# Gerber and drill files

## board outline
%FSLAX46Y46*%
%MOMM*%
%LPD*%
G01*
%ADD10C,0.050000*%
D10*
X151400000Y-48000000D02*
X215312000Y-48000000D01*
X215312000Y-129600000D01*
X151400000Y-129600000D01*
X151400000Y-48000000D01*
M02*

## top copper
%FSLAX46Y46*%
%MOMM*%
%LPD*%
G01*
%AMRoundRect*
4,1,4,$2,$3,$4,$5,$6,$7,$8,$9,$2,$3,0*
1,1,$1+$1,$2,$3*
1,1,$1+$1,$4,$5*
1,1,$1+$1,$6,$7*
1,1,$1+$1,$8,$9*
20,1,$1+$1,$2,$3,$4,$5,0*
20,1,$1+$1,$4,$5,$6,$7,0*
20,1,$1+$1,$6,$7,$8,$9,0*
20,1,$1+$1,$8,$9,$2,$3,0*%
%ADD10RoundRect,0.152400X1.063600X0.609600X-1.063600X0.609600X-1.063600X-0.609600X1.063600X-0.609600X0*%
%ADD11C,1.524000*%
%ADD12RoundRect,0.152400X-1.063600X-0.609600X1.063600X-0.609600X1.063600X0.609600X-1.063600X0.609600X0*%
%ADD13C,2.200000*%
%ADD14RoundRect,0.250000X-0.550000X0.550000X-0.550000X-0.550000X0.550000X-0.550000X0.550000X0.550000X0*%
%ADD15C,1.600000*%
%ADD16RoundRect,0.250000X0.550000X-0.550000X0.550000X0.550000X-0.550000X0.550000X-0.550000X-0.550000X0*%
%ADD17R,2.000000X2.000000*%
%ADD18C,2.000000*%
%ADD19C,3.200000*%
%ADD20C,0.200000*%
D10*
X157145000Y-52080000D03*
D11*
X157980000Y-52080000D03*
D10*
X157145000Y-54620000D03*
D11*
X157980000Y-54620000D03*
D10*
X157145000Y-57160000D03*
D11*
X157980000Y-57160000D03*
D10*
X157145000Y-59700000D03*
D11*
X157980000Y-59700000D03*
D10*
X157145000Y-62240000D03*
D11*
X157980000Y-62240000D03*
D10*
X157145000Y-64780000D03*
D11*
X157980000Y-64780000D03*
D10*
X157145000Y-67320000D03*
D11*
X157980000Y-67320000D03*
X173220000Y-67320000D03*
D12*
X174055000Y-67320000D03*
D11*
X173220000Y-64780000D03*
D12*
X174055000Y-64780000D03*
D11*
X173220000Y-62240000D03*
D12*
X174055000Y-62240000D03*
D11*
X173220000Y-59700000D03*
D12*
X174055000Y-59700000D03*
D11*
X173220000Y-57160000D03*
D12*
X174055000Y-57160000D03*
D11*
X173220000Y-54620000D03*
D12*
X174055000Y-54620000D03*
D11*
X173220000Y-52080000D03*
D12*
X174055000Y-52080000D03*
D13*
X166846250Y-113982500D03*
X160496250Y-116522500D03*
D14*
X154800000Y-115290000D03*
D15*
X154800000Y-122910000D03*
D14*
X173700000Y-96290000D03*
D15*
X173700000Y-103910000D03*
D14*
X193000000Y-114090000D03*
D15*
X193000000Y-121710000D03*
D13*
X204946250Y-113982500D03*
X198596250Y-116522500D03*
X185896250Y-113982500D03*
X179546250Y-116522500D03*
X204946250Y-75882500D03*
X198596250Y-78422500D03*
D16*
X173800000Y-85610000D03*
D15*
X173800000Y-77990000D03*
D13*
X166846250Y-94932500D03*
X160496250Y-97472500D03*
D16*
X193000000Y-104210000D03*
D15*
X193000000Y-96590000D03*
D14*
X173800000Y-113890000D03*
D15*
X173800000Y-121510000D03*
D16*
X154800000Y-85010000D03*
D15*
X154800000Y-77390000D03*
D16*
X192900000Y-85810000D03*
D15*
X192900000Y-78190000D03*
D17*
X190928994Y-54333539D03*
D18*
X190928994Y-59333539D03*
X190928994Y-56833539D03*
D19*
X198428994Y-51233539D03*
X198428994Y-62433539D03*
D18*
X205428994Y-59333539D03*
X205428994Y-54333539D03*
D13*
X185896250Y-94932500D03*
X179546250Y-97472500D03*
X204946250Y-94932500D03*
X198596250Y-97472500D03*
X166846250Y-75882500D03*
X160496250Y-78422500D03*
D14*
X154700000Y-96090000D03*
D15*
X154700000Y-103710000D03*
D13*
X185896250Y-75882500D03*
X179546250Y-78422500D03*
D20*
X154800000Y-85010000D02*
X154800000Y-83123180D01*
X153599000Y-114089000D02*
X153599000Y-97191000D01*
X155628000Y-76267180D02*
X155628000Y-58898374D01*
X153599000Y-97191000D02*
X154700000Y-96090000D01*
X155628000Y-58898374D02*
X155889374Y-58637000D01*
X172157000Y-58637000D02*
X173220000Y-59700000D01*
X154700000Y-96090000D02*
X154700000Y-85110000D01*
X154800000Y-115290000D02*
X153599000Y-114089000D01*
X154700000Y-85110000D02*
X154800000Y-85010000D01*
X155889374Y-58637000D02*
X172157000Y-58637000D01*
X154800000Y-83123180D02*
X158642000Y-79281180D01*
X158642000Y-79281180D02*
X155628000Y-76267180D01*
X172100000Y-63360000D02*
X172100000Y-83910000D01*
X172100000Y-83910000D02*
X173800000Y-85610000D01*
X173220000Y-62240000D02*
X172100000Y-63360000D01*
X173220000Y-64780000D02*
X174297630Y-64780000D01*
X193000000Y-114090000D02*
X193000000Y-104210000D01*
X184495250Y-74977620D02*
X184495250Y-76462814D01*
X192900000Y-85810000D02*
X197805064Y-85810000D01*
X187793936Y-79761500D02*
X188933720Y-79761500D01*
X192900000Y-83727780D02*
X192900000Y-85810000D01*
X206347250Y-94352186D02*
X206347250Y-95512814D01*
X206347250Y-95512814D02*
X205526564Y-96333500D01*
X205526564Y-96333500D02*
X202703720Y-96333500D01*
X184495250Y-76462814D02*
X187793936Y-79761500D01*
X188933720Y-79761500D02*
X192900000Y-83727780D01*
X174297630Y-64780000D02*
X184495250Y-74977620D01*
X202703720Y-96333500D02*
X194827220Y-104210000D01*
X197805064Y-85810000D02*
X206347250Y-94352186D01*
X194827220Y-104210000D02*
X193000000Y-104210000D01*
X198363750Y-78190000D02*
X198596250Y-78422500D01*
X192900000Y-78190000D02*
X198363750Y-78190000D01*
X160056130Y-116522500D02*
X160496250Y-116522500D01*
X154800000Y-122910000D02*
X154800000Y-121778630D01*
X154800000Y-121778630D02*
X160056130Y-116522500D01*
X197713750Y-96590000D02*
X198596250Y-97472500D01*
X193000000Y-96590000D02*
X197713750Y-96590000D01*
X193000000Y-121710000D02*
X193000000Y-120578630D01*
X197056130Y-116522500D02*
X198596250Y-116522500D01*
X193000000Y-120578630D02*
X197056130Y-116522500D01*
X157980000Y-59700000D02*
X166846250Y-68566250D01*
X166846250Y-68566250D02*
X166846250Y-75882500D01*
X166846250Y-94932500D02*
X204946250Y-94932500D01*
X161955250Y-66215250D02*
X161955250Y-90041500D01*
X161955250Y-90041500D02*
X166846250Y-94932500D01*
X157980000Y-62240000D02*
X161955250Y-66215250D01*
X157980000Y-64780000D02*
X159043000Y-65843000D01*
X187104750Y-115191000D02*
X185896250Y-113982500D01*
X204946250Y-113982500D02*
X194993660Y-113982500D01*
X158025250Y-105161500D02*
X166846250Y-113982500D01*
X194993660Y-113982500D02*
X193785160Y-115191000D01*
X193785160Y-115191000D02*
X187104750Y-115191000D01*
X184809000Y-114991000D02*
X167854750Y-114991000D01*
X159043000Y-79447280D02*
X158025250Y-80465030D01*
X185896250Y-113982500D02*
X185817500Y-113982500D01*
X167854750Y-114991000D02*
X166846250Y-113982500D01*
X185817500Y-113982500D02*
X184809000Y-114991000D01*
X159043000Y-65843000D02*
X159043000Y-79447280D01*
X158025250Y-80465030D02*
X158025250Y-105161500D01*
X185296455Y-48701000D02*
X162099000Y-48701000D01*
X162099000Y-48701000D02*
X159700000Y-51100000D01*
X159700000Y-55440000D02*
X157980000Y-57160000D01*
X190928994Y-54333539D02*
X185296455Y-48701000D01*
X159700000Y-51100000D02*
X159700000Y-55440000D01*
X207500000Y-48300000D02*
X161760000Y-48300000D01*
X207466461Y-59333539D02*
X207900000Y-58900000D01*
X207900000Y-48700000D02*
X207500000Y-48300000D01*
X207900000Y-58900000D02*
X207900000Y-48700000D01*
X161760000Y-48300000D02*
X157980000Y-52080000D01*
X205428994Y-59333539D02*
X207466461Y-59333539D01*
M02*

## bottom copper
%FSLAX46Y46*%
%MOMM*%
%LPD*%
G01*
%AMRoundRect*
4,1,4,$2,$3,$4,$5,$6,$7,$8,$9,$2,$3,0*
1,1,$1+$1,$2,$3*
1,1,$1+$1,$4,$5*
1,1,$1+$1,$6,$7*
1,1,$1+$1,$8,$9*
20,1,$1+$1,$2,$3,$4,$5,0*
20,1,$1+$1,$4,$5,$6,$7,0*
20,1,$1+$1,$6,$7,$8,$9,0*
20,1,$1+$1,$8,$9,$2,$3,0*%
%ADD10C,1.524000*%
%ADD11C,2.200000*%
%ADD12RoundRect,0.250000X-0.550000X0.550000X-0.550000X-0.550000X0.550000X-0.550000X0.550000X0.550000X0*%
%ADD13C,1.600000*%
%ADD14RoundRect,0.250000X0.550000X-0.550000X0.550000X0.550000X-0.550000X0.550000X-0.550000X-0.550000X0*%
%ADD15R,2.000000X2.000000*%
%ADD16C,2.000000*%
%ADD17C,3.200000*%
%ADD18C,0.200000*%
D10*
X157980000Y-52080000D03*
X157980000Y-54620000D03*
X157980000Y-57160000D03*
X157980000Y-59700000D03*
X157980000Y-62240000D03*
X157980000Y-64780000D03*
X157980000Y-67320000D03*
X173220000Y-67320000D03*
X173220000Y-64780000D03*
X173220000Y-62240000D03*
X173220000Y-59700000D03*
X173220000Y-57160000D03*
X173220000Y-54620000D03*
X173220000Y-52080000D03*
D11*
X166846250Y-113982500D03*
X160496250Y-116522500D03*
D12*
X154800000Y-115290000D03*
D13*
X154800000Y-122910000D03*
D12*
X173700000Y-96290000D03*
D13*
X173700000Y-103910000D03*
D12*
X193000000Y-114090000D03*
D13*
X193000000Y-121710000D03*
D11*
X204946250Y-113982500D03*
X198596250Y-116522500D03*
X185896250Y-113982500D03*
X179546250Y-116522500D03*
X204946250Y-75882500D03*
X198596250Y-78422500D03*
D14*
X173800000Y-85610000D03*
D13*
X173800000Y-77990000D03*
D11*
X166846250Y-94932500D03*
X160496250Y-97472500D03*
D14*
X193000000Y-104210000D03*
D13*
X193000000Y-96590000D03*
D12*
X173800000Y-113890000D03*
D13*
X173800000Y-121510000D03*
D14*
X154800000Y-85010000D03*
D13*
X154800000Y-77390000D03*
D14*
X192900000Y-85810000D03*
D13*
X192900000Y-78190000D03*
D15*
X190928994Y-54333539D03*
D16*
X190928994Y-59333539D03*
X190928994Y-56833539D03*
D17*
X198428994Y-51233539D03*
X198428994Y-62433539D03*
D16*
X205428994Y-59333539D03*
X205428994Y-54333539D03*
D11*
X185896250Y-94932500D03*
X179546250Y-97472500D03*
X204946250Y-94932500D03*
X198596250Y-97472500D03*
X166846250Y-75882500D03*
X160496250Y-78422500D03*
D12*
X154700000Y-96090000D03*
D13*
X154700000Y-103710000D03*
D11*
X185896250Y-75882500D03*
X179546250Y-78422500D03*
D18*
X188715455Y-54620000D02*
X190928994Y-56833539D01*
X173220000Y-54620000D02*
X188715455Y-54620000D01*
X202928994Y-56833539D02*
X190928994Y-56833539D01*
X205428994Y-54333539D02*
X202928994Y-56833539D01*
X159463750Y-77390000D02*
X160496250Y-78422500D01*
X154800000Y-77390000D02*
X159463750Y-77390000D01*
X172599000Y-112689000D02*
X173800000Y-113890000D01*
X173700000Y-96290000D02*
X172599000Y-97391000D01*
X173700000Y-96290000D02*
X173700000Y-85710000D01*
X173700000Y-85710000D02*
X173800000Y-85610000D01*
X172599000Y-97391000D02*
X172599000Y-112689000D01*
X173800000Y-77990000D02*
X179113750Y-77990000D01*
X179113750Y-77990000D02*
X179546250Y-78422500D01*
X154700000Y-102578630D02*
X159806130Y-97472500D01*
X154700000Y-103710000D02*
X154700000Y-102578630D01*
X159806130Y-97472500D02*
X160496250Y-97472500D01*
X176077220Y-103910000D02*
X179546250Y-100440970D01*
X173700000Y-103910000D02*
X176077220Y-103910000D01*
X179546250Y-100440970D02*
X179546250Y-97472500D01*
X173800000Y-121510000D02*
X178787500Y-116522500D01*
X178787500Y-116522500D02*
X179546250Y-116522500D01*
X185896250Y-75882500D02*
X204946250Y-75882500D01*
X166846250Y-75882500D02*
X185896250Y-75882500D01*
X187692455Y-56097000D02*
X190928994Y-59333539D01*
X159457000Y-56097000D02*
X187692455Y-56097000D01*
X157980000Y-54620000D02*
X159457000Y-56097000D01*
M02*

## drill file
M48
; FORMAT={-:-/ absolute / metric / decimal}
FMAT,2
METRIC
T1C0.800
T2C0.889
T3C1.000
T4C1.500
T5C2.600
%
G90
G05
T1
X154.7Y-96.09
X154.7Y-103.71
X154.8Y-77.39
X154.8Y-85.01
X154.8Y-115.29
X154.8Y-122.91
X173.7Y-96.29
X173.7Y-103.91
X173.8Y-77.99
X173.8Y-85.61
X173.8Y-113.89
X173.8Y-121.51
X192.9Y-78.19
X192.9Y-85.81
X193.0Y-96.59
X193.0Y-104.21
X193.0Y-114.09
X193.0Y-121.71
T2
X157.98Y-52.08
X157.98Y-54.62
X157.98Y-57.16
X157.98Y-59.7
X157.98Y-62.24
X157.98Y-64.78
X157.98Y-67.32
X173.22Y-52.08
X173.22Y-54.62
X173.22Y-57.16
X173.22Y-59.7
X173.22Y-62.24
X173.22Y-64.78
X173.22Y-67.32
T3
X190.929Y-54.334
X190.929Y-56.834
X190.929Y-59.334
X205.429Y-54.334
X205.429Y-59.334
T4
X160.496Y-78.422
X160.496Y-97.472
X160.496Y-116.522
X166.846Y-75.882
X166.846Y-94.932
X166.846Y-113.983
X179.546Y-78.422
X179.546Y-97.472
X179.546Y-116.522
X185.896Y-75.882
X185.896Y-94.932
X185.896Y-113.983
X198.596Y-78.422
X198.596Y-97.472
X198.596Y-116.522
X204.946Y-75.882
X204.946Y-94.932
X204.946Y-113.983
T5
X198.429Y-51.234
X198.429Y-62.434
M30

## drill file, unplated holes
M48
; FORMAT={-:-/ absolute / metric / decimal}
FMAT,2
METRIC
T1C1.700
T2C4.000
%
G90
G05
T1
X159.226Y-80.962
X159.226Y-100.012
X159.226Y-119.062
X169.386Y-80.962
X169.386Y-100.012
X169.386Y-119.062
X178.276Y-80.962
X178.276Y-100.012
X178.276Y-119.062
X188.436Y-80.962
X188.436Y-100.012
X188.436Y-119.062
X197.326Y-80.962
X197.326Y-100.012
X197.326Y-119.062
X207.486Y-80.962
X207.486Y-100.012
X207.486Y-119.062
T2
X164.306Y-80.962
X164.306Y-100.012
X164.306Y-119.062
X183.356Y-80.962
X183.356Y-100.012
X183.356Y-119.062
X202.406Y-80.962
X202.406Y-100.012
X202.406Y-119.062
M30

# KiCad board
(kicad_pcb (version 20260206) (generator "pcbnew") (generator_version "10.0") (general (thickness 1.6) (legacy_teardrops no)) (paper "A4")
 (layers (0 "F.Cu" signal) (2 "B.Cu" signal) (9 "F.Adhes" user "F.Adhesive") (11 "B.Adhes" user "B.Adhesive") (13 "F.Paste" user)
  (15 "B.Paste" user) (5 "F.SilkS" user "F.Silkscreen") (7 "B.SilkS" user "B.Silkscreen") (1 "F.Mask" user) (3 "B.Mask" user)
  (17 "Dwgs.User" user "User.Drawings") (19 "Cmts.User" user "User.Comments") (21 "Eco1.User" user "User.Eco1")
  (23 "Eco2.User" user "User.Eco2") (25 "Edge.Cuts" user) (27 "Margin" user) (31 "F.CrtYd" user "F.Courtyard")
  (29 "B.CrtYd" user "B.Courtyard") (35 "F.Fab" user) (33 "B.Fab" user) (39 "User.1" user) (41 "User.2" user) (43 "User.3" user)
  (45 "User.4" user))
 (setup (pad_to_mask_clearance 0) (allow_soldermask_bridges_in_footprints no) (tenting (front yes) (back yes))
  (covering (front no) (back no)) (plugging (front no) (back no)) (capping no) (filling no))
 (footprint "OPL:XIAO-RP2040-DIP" (layer "F.Cu") (at 165.6 59.7)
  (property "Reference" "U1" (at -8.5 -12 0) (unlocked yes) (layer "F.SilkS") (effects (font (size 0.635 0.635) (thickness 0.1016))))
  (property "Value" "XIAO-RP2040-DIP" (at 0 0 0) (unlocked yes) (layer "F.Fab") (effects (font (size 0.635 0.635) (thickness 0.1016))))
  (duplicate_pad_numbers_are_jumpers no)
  (pad "1" smd roundrect (at -8.455 -7.62 180) (size 2.432 1.524) (layers "F.Cu" "F.Mask") (roundrect_rratio 0.1)
   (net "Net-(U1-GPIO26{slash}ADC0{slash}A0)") (thermal_bridge_angle 45))
  (pad "1" thru_hole circle (at -7.62 -7.62 180) (size 1.524 1.524) (drill 0.889) (layers "*.Cu" "*.Mask") (remove_unused_layers no)
   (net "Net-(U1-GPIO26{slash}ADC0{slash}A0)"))
  (pad "2" smd roundrect (at -8.455 -5.08 180) (size 2.432 1.524) (layers "F.Cu" "F.Mask") (roundrect_rratio 0.1)
   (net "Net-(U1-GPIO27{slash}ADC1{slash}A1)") (thermal_bridge_angle 45))
  (pad "2" thru_hole circle (at -7.62 -5.08 180) (size 1.524 1.524) (drill 0.889) (layers "*.Cu" "*.Mask") (remove_unused_layers no)
   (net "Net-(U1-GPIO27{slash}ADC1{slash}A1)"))
  (pad "3" smd roundrect (at -8.455 -2.54 180) (size 2.432 1.524) (layers "F.Cu" "F.Mask") (roundrect_rratio 0.1)
   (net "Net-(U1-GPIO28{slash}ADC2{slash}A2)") (thermal_bridge_angle 45))
  (pad "3" thru_hole circle (at -7.62 -2.54 180) (size 1.524 1.524) (drill 0.889) (layers "*.Cu" "*.Mask") (remove_unused_layers no)
   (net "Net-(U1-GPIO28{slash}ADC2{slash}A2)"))
  (pad "4" smd roundrect (at -8.455 0 180) (size 2.432 1.524) (layers "F.Cu" "F.Mask") (roundrect_rratio 0.1) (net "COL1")
   (thermal_bridge_angle 45))
  (pad "4" thru_hole circle (at -7.62 0 180) (size 1.524 1.524) (drill 0.889) (layers "*.Cu" "*.Mask") (remove_unused_layers no)
   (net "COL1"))
  (pad "5" smd roundrect (at -8.455 2.54 180) (size 2.432 1.524) (layers "F.Cu" "F.Mask") (roundrect_rratio 0.1) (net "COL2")
   (thermal_bridge_angle 45))
  (pad "5" thru_hole circle (at -7.62 2.54 180) (size 1.524 1.524) (drill 0.889) (layers "*.Cu" "*.Mask") (remove_unused_layers no)
   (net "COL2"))
  (pad "6" smd roundrect (at -8.455 5.08 180) (size 2.432 1.524) (layers "F.Cu" "F.Mask") (roundrect_rratio 0.1) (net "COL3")
   (thermal_bridge_angle 45))
  (pad "6" thru_hole circle (at -7.62 5.08 180) (size 1.524 1.524) (drill 0.889) (layers "*.Cu" "*.Mask") (remove_unused_layers no)
   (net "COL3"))
  (pad "7" smd roundrect (at -8.455 7.62 180) (size 2.432 1.524) (layers "F.Cu" "F.Mask") (roundrect_rratio 0.1)
   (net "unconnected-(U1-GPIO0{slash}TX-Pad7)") (thermal_bridge_angle 45))
  (pad "7" thru_hole circle (at -7.62 7.62 180) (size 1.524 1.524) (drill 0.889) (layers "*.Cu" "*.Mask") (remove_unused_layers no)
   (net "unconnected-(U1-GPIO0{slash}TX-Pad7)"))
  (pad "8" thru_hole circle (at 7.62 7.62) (size 1.524 1.524) (drill 0.889) (layers "*.Cu" "*.Mask") (remove_unused_layers no)
   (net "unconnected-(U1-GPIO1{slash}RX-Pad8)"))
  (pad "8" smd roundrect (at 8.455 7.62) (size 2.432 1.524) (layers "F.Cu" "F.Mask") (roundrect_rratio 0.1)
   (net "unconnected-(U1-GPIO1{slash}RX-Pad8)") (thermal_bridge_angle 45))
  (pad "9" thru_hole circle (at 7.62 5.08) (size 1.524 1.524) (drill 0.889) (layers "*.Cu" "*.Mask") (remove_unused_layers no) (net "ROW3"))
  (pad "9" smd roundrect (at 8.455 5.08) (size 2.432 1.524) (layers "F.Cu" "F.Mask") (roundrect_rratio 0.1) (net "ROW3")
   (thermal_bridge_angle 45))
  (pad "10" thru_hole circle (at 7.62 2.54) (size 1.524 1.524) (drill 0.889) (layers "*.Cu" "*.Mask") (remove_unused_layers no) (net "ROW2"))
  (pad "10" smd roundrect (at 8.455 2.54) (size 2.432 1.524) (layers "F.Cu" "F.Mask") (roundrect_rratio 0.1) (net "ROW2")
   (thermal_bridge_angle 45))
  (pad "11" thru_hole circle (at 7.62 0) (size 1.524 1.524) (drill 0.889) (layers "*.Cu" "*.Mask") (remove_unused_layers no) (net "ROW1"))
  (pad "11" smd roundrect (at 8.455 0) (size 2.432 1.524) (layers "F.Cu" "F.Mask") (roundrect_rratio 0.1) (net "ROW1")
   (thermal_bridge_angle 45))
  (pad "12" thru_hole circle (at 7.62 -2.54) (size 1.524 1.524) (drill 0.889) (layers "*.Cu" "*.Mask") (remove_unused_layers no)
   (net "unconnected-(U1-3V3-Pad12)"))
  (pad "12" smd roundrect (at 8.455 -2.54) (size 2.432 1.524) (layers "F.Cu" "F.Mask") (roundrect_rratio 0.1)
   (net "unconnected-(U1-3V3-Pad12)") (thermal_bridge_angle 45))
  (pad "13" thru_hole circle (at 7.62 -5.08) (size 1.524 1.524) (drill 0.889) (layers "*.Cu" "*.Mask") (remove_unused_layers no) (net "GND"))
  (pad "13" smd roundrect (at 8.455 -5.08) (size 2.432 1.524) (layers "F.Cu" "F.Mask") (roundrect_rratio 0.1) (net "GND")
   (thermal_bridge_angle 45))
  (pad "14" thru_hole circle (at 7.62 -7.62) (size 1.524 1.524) (drill 0.889) (layers "*.Cu" "*.Mask") (remove_unused_layers no) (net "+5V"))
  (pad "14" smd roundrect (at 8.455 -7.62) (size 2.432 1.524) (layers "F.Cu" "F.Mask") (roundrect_rratio 0.1) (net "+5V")
   (thermal_bridge_angle 45)))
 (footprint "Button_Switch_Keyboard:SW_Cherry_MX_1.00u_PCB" (layer "F.Cu") (at 166.84625 113.9825)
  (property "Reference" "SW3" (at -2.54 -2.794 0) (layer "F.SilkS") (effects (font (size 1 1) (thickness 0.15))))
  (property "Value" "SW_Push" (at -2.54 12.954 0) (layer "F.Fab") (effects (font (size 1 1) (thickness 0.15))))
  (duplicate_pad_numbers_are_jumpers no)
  (pad "" np_thru_hole circle (at -7.62 5.08) (size 1.7 1.7) (drill 1.7) (layers "*.Cu" "*.Mask"))
  (pad "" np_thru_hole circle (at -2.54 5.08) (size 4 4) (drill 4) (layers "*.Cu" "*.Mask"))
  (pad "" np_thru_hole circle (at 2.54 5.08) (size 1.7 1.7) (drill 1.7) (layers "*.Cu" "*.Mask"))
  (pad "1" thru_hole circle (at 0 0) (size 2.2 2.2) (drill 1.5) (layers "*.Cu" "*.Mask") (remove_unused_layers no) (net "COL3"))
  (pad "2" thru_hole circle (at -6.35 2.54) (size 2.2 2.2) (drill 1.5) (layers "*.Cu" "*.Mask") (remove_unused_layers no) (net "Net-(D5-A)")))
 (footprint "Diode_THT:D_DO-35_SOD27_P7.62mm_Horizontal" (layer "F.Cu") (at 154.8 115.29 -90)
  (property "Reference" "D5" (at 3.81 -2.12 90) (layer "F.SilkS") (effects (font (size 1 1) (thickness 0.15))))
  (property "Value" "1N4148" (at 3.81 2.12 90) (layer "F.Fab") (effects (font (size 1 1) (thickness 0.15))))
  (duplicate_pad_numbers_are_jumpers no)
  (pad "1" thru_hole roundrect (at 0 0 270) (size 1.6 1.6) (drill 0.8) (layers "*.Cu" "*.Mask") (remove_unused_layers no)
   (roundrect_rratio 0.15625) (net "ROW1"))
  (pad "2" thru_hole circle (at 7.62 0 270) (size 1.6 1.6) (drill 0.8) (layers "*.Cu" "*.Mask") (remove_unused_layers no) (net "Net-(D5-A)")))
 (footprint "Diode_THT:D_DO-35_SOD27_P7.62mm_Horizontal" (layer "F.Cu") (at 173.7 96.29 -90)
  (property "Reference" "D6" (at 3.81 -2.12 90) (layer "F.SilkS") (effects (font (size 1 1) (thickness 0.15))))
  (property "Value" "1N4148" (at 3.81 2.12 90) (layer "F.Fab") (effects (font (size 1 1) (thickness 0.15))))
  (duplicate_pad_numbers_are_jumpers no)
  (pad "1" thru_hole roundrect (at 0 0 270) (size 1.6 1.6) (drill 0.8) (layers "*.Cu" "*.Mask") (remove_unused_layers no)
   (roundrect_rratio 0.15625) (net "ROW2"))
  (pad "2" thru_hole circle (at 7.62 0 270) (size 1.6 1.6) (drill 0.8) (layers "*.Cu" "*.Mask") (remove_unused_layers no) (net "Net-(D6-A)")))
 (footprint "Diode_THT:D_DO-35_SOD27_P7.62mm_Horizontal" (layer "F.Cu") (at 193 114.09 -90)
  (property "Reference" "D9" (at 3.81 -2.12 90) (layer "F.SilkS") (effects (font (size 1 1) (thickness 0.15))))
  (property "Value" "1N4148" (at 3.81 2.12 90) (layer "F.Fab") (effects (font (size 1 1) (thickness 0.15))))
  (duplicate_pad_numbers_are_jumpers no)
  (pad "1" thru_hole roundrect (at 0 0 270) (size 1.6 1.6) (drill 0.8) (layers "*.Cu" "*.Mask") (remove_unused_layers no)
   (roundrect_rratio 0.15625) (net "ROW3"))
  (pad "2" thru_hole circle (at 7.62 0 270) (size 1.6 1.6) (drill 0.8) (layers "*.Cu" "*.Mask") (remove_unused_layers no) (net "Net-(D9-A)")))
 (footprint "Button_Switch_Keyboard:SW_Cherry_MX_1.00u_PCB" (layer "F.Cu") (at 204.94625 113.9825)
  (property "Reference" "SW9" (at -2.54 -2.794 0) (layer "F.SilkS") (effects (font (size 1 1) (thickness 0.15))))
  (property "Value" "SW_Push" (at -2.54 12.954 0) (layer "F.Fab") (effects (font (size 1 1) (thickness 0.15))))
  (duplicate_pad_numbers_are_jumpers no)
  (pad "" np_thru_hole circle (at -7.62 5.08) (size 1.7 1.7) (drill 1.7) (layers "*.Cu" "*.Mask"))
  (pad "" np_thru_hole circle (at -2.54 5.08) (size 4 4) (drill 4) (layers "*.Cu" "*.Mask"))
  (pad "" np_thru_hole circle (at 2.54 5.08) (size 1.7 1.7) (drill 1.7) (layers "*.Cu" "*.Mask"))
  (pad "1" thru_hole circle (at 0 0) (size 2.2 2.2) (drill 1.5) (layers "*.Cu" "*.Mask") (remove_unused_layers no) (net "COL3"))
  (pad "2" thru_hole circle (at -6.35 2.54) (size 2.2 2.2) (drill 1.5) (layers "*.Cu" "*.Mask") (remove_unused_layers no) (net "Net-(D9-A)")))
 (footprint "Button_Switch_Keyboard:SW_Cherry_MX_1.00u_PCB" (layer "F.Cu") (at 185.89625 113.9825)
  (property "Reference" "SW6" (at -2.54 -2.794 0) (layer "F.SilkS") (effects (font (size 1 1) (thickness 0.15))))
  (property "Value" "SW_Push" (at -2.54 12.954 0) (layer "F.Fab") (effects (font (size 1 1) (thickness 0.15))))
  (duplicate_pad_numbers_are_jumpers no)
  (pad "" np_thru_hole circle (at -7.62 5.08) (size 1.7 1.7) (drill 1.7) (layers "*.Cu" "*.Mask"))
  (pad "" np_thru_hole circle (at -2.54 5.08) (size 4 4) (drill 4) (layers "*.Cu" "*.Mask"))
  (pad "" np_thru_hole circle (at 2.54 5.08) (size 1.7 1.7) (drill 1.7) (layers "*.Cu" "*.Mask"))
  (pad "1" thru_hole circle (at 0 0) (size 2.2 2.2) (drill 1.5) (layers "*.Cu" "*.Mask") (remove_unused_layers no) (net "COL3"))
  (pad "2" thru_hole circle (at -6.35 2.54) (size 2.2 2.2) (drill 1.5) (layers "*.Cu" "*.Mask") (remove_unused_layers no) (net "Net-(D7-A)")))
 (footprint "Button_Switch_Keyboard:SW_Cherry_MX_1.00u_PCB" (layer "F.Cu") (at 204.94625 75.8825)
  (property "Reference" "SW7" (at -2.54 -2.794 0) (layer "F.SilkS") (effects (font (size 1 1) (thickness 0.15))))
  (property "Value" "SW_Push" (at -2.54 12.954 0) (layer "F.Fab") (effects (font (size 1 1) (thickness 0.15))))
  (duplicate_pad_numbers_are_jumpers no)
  (pad "" np_thru_hole circle (at -7.62 5.08) (size 1.7 1.7) (drill 1.7) (layers "*.Cu" "*.Mask"))
  (pad "" np_thru_hole circle (at -2.54 5.08) (size 4 4) (drill 4) (layers "*.Cu" "*.Mask"))
  (pad "" np_thru_hole circle (at 2.54 5.08) (size 1.7 1.7) (drill 1.7) (layers "*.Cu" "*.Mask"))
  (pad "1" thru_hole circle (at 0 0) (size 2.2 2.2) (drill 1.5) (layers "*.Cu" "*.Mask") (remove_unused_layers no) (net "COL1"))
  (pad "2" thru_hole circle (at -6.35 2.54) (size 2.2 2.2) (drill 1.5) (layers "*.Cu" "*.Mask") (remove_unused_layers no) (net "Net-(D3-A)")))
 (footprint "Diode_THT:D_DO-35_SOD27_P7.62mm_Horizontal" (layer "F.Cu") (at 173.8 85.61 90)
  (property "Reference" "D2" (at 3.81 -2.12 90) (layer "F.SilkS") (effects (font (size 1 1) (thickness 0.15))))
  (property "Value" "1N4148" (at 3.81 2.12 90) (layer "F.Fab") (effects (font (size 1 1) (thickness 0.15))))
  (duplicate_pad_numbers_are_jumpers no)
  (pad "1" thru_hole roundrect (at 0 0 90) (size 1.6 1.6) (drill 0.8) (layers "*.Cu" "*.Mask") (remove_unused_layers no)
   (roundrect_rratio 0.15625) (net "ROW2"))
  (pad "2" thru_hole circle (at 7.62 0 90) (size 1.6 1.6) (drill 0.8) (layers "*.Cu" "*.Mask") (remove_unused_layers no) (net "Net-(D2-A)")))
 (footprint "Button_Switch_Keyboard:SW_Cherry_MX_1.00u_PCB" (layer "F.Cu") (at 166.84625 94.9325)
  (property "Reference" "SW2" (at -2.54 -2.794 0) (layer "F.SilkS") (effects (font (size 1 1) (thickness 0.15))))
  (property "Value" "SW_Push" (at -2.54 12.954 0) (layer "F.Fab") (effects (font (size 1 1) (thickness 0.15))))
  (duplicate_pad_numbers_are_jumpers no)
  (pad "" np_thru_hole circle (at -7.62 5.08) (size 1.7 1.7) (drill 1.7) (layers "*.Cu" "*.Mask"))
  (pad "" np_thru_hole circle (at -2.54 5.08) (size 4 4) (drill 4) (layers "*.Cu" "*.Mask"))
  (pad "" np_thru_hole circle (at 2.54 5.08) (size 1.7 1.7) (drill 1.7) (layers "*.Cu" "*.Mask"))
  (pad "1" thru_hole circle (at 0 0) (size 2.2 2.2) (drill 1.5) (layers "*.Cu" "*.Mask") (remove_unused_layers no) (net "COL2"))
  (pad "2" thru_hole circle (at -6.35 2.54) (size 2.2 2.2) (drill 1.5) (layers "*.Cu" "*.Mask") (remove_unused_layers no) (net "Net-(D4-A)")))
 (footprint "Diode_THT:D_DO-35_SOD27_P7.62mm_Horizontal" (layer "F.Cu") (at 193 104.21 90)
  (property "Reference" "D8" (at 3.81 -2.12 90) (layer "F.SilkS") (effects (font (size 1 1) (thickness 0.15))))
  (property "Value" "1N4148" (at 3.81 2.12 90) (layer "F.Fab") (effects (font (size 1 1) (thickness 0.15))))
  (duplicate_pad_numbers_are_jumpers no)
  (pad "1" thru_hole roundrect (at 0 0 90) (size 1.6 1.6) (drill 0.8) (layers "*.Cu" "*.Mask") (remove_unused_layers no)
   (roundrect_rratio 0.15625) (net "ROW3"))
  (pad "2" thru_hole circle (at 7.62 0 90) (size 1.6 1.6) (drill 0.8) (layers "*.Cu" "*.Mask") (remove_unused_layers no) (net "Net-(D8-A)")))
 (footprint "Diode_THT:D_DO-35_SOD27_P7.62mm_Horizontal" (layer "F.Cu") (at 173.8 113.89 -90)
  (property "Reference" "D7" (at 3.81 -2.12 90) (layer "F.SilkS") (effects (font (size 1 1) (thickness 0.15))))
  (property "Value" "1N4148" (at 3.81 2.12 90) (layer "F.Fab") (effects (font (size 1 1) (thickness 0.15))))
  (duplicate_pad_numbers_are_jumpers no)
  (pad "1" thru_hole roundrect (at 0 0 270) (size 1.6 1.6) (drill 0.8) (layers "*.Cu" "*.Mask") (remove_unused_layers no)
   (roundrect_rratio 0.15625) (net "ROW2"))
  (pad "2" thru_hole circle (at 7.62 0 270) (size 1.6 1.6) (drill 0.8) (layers "*.Cu" "*.Mask") (remove_unused_layers no) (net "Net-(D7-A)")))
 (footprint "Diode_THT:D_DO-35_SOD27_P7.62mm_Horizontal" (layer "F.Cu") (at 154.8 85.01 90)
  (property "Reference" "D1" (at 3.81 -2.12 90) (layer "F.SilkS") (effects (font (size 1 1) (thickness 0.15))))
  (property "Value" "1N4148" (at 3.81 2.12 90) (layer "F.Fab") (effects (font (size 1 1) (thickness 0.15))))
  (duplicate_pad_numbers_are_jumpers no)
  (pad "1" thru_hole roundrect (at 0 0 90) (size 1.6 1.6) (drill 0.8) (layers "*.Cu" "*.Mask") (remove_unused_layers no)
   (roundrect_rratio 0.15625) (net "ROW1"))
  (pad "2" thru_hole circle (at 7.62 0 90) (size 1.6 1.6) (drill 0.8) (layers "*.Cu" "*.Mask") (remove_unused_layers no) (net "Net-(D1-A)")))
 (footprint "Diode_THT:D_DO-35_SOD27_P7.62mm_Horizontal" (layer "F.Cu") (at 192.9 85.81 90)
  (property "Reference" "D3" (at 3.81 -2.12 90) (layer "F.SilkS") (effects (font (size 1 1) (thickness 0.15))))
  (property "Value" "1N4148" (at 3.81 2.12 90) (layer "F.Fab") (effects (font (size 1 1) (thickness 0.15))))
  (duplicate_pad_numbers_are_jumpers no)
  (pad "1" thru_hole roundrect (at 0 0 90) (size 1.6 1.6) (drill 0.8) (layers "*.Cu" "*.Mask") (remove_unused_layers no)
   (roundrect_rratio 0.15625) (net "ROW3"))
  (pad "2" thru_hole circle (at 7.62 0 90) (size 1.6 1.6) (drill 0.8) (layers "*.Cu" "*.Mask") (remove_unused_layers no) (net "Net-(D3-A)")))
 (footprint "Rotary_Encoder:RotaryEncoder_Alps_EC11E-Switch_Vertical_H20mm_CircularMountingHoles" (layer "F.Cu") (at 190.928994 54.333539)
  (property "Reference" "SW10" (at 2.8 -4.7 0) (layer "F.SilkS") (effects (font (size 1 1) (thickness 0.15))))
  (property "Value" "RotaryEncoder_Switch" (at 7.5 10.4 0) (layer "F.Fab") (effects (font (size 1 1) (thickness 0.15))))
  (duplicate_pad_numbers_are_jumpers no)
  (pad "A" thru_hole rect (at 0 0) (size 2 2) (drill 1) (layers "*.Cu" "*.Mask") (remove_unused_layers no)
   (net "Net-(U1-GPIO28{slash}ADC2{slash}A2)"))
  (pad "B" thru_hole circle (at 0 5) (size 2 2) (drill 1) (layers "*.Cu" "*.Mask") (remove_unused_layers no)
   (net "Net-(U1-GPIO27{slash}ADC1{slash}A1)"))
  (pad "C" thru_hole circle (at 0 2.5) (size 2 2) (drill 1) (layers "*.Cu" "*.Mask") (remove_unused_layers no) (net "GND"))
  (pad "MP" thru_hole circle (at 7.5 -3.1) (size 3.2 3.2) (drill 2.6) (layers "*.Cu" "*.Mask") (remove_unused_layers no))
  (pad "MP" thru_hole circle (at 7.5 8.1) (size 3.2 3.2) (drill 2.6) (layers "*.Cu" "*.Mask") (remove_unused_layers no))
  (pad "S1" thru_hole circle (at 14.5 5) (size 2 2) (drill 1) (layers "*.Cu" "*.Mask") (remove_unused_layers no)
   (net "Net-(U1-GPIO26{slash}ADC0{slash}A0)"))
  (pad "S2" thru_hole circle (at 14.5 0) (size 2 2) (drill 1) (layers "*.Cu" "*.Mask") (remove_unused_layers no) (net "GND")))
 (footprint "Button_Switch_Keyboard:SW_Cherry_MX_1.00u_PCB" (layer "F.Cu") (at 185.89625 94.9325)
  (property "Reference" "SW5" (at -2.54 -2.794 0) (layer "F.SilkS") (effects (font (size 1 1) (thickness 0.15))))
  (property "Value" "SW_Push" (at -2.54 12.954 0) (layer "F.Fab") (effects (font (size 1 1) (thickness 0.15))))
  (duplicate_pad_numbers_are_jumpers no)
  (pad "" np_thru_hole circle (at -7.62 5.08) (size 1.7 1.7) (drill 1.7) (layers "*.Cu" "*.Mask"))
  (pad "" np_thru_hole circle (at -2.54 5.08) (size 4 4) (drill 4) (layers "*.Cu" "*.Mask"))
  (pad "" np_thru_hole circle (at 2.54 5.08) (size 1.7 1.7) (drill 1.7) (layers "*.Cu" "*.Mask"))
  (pad "1" thru_hole circle (at 0 0) (size 2.2 2.2) (drill 1.5) (layers "*.Cu" "*.Mask") (remove_unused_layers no) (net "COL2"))
  (pad "2" thru_hole circle (at -6.35 2.54) (size 2.2 2.2) (drill 1.5) (layers "*.Cu" "*.Mask") (remove_unused_layers no) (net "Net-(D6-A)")))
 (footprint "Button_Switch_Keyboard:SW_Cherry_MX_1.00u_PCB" (layer "F.Cu") (at 204.94625 94.9325)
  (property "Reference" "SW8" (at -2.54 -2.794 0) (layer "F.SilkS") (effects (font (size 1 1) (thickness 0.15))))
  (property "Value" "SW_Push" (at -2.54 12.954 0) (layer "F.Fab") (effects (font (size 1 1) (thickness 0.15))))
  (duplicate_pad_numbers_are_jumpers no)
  (pad "" np_thru_hole circle (at -7.62 5.08) (size 1.7 1.7) (drill 1.7) (layers "*.Cu" "*.Mask"))
  (pad "" np_thru_hole circle (at -2.54 5.08) (size 4 4) (drill 4) (layers "*.Cu" "*.Mask"))
  (pad "" np_thru_hole circle (at 2.54 5.08) (size 1.7 1.7) (drill 1.7) (layers "*.Cu" "*.Mask"))
  (pad "1" thru_hole circle (at 0 0) (size 2.2 2.2) (drill 1.5) (layers "*.Cu" "*.Mask") (remove_unused_layers no) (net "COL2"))
  (pad "2" thru_hole circle (at -6.35 2.54) (size 2.2 2.2) (drill 1.5) (layers "*.Cu" "*.Mask") (remove_unused_layers no) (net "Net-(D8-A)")))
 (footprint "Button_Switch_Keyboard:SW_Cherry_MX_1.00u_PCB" (layer "F.Cu") (at 166.84625 75.8825)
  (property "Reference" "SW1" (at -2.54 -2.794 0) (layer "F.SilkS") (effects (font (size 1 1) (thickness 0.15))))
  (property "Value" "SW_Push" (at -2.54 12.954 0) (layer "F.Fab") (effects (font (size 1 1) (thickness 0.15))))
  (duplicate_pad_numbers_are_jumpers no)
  (pad "" np_thru_hole circle (at -7.62 5.08) (size 1.7 1.7) (drill 1.7) (layers "*.Cu" "*.Mask"))
  (pad "" np_thru_hole circle (at -2.54 5.08) (size 4 4) (drill 4) (layers "*.Cu" "*.Mask"))
  (pad "" np_thru_hole circle (at 2.54 5.08) (size 1.7 1.7) (drill 1.7) (layers "*.Cu" "*.Mask"))
  (pad "1" thru_hole circle (at 0 0) (size 2.2 2.2) (drill 1.5) (layers "*.Cu" "*.Mask") (remove_unused_layers no) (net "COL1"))
  (pad "2" thru_hole circle (at -6.35 2.54) (size 2.2 2.2) (drill 1.5) (layers "*.Cu" "*.Mask") (remove_unused_layers no) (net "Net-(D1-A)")))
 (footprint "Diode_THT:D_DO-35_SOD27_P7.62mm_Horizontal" (layer "F.Cu") (at 154.7 96.09 -90)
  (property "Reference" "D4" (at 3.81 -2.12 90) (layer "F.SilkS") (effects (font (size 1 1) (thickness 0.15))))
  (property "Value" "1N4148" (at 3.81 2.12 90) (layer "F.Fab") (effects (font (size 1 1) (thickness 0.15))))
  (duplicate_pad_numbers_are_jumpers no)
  (pad "1" thru_hole roundrect (at 0 0 270) (size 1.6 1.6) (drill 0.8) (layers "*.Cu" "*.Mask") (remove_unused_layers no)
   (roundrect_rratio 0.15625) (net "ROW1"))
  (pad "2" thru_hole circle (at 7.62 0 270) (size 1.6 1.6) (drill 0.8) (layers "*.Cu" "*.Mask") (remove_unused_layers no) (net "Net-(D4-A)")))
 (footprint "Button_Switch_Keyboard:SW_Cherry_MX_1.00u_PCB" (layer "F.Cu") (at 185.89625 75.8825)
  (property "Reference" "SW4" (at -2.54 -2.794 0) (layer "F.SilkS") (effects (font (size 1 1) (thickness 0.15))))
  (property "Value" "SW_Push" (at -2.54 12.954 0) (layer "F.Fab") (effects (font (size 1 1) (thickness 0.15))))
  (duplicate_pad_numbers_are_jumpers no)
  (pad "" np_thru_hole circle (at -7.62 5.08) (size 1.7 1.7) (drill 1.7) (layers "*.Cu" "*.Mask"))
  (pad "" np_thru_hole circle (at -2.54 5.08) (size 4 4) (drill 4) (layers "*.Cu" "*.Mask"))
  (pad "" np_thru_hole circle (at 2.54 5.08) (size 1.7 1.7) (drill 1.7) (layers "*.Cu" "*.Mask"))
  (pad "1" thru_hole circle (at 0 0) (size 2.2 2.2) (drill 1.5) (layers "*.Cu" "*.Mask") (remove_unused_layers no) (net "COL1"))
  (pad "2" thru_hole circle (at -6.35 2.54) (size 2.2 2.2) (drill 1.5) (layers "*.Cu" "*.Mask") (remove_unused_layers no) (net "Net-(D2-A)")))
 (gr_rect (start 151.4 48) (end 215.312 129.6) (stroke (width 0.05) (type default)) (fill no) (layer "Edge.Cuts"))
 (segment (start 188.715455 54.62) (end 190.928994 56.833539) (width 0.2) (layer "B.Cu") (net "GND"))
 (segment (start 173.22 54.62) (end 188.715455 54.62) (width 0.2) (layer "B.Cu") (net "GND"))
 (segment (start 202.928994 56.833539) (end 190.928994 56.833539) (width 0.2) (layer "B.Cu") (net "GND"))
 (segment (start 205.428994 54.333539) (end 202.928994 56.833539) (width 0.2) (layer "B.Cu") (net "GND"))
 (segment (start 154.8 85.01) (end 154.8 83.12318) (width 0.2) (layer "F.Cu") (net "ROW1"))
 (segment (start 153.599 114.089) (end 153.599 97.191) (width 0.2) (layer "F.Cu") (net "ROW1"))
 (segment (start 155.628 76.26718) (end 155.628 58.898374) (width 0.2) (layer "F.Cu") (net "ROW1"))
 (segment (start 153.599 97.191) (end 154.7 96.09) (width 0.2) (layer "F.Cu") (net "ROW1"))
 (segment (start 155.628 58.898374) (end 155.889374 58.637) (width 0.2) (layer "F.Cu") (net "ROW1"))
 (segment (start 172.157 58.637) (end 173.22 59.7) (width 0.2) (layer "F.Cu") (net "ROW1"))
 (segment (start 154.7 96.09) (end 154.7 85.11) (width 0.2) (layer "F.Cu") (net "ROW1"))
 (segment (start 154.8 115.29) (end 153.599 114.089) (width 0.2) (layer "F.Cu") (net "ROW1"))
 (segment (start 154.7 85.11) (end 154.8 85.01) (width 0.2) (layer "F.Cu") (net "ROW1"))
 (segment (start 155.889374 58.637) (end 172.157 58.637) (width 0.2) (layer "F.Cu") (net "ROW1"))
 (segment (start 154.8 83.12318) (end 158.642 79.28118) (width 0.2) (layer "F.Cu") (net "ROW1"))
 (segment (start 158.642 79.28118) (end 155.628 76.26718) (width 0.2) (layer "F.Cu") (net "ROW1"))
 (segment (start 159.46375 77.39) (end 160.49625 78.4225) (width 0.2) (layer "B.Cu") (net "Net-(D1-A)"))
 (segment (start 154.8 77.39) (end 159.46375 77.39) (width 0.2) (layer "B.Cu") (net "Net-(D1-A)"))
 (segment (start 172.1 63.36) (end 172.1 83.91) (width 0.2) (layer "F.Cu") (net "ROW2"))
 (segment (start 172.1 83.91) (end 173.8 85.61) (width 0.2) (layer "F.Cu") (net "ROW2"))
 (segment (start 173.22 62.24) (end 172.1 63.36) (width 0.2) (layer "F.Cu") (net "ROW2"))
 (segment (start 172.599 112.689) (end 173.8 113.89) (width 0.2) (layer "B.Cu") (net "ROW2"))
 (segment (start 173.7 96.29) (end 172.599 97.391) (width 0.2) (layer "B.Cu") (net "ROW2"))
 (segment (start 173.7 96.29) (end 173.7 85.71) (width 0.2) (layer "B.Cu") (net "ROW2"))
 (segment (start 173.7 85.71) (end 173.8 85.61) (width 0.2) (layer "B.Cu") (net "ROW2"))
 (segment (start 172.599 97.391) (end 172.599 112.689) (width 0.2) (layer "B.Cu") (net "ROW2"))
 (segment (start 173.8 77.99) (end 179.11375 77.99) (width 0.2) (layer "B.Cu") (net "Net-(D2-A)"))
 (segment (start 179.11375 77.99) (end 179.54625 78.4225) (width 0.2) (layer "B.Cu") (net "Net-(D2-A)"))
 (segment (start 173.22 64.78) (end 174.29763 64.78) (width 0.2) (layer "F.Cu") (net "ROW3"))
 (segment (start 193 114.09) (end 193 104.21) (width 0.2) (layer "F.Cu") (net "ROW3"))
 (segment (start 184.49525 74.97762) (end 184.49525 76.462814) (width 0.2) (layer "F.Cu") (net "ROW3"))
 (segment (start 192.9 85.81) (end 197.805064 85.81) (width 0.2) (layer "F.Cu") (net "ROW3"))
 (segment (start 187.793936 79.7615) (end 188.93372 79.7615) (width 0.2) (layer "F.Cu") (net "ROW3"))
 (segment (start 192.9 83.72778) (end 192.9 85.81) (width 0.2) (layer "F.Cu") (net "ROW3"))
 (segment (start 206.34725 94.352186) (end 206.34725 95.512814) (width 0.2) (layer "F.Cu") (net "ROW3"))
 (segment (start 206.34725 95.512814) (end 205.526564 96.3335) (width 0.2) (layer "F.Cu") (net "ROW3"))
 (segment (start 205.526564 96.3335) (end 202.70372 96.3335) (width 0.2) (layer "F.Cu") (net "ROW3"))
 (segment (start 184.49525 76.462814) (end 187.793936 79.7615) (width 0.2) (layer "F.Cu") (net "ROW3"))
 (segment (start 188.93372 79.7615) (end 192.9 83.72778) (width 0.2) (layer "F.Cu") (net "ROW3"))
 (segment (start 174.29763 64.78) (end 184.49525 74.97762) (width 0.2) (layer "F.Cu") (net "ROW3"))
 (segment (start 202.70372 96.3335) (end 194.82722 104.21) (width 0.2) (layer "F.Cu") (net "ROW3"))
 (segment (start 197.805064 85.81) (end 206.34725 94.352186) (width 0.2) (layer "F.Cu") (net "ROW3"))
 (segment (start 194.82722 104.21) (end 193 104.21) (width 0.2) (layer "F.Cu") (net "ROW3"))
 (segment (start 198.36375 78.19) (end 198.59625 78.4225) (width 0.2) (layer "F.Cu") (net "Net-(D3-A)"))
 (segment (start 192.9 78.19) (end 198.36375 78.19) (width 0.2) (layer "F.Cu") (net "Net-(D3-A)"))
 (segment (start 154.7 102.57863) (end 159.80613 97.4725) (width 0.2) (layer "B.Cu") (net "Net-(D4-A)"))
 (segment (start 154.7 103.71) (end 154.7 102.57863) (width 0.2) (layer "B.Cu") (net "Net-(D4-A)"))
 (segment (start 159.80613 97.4725) (end 160.49625 97.4725) (width 0.2) (layer "B.Cu") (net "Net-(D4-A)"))
 (segment (start 160.05613 116.5225) (end 160.49625 116.5225) (width 0.2) (layer "F.Cu") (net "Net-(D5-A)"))
 (segment (start 154.8 122.91) (end 154.8 121.77863) (width 0.2) (layer "F.Cu") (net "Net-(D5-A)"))
 (segment (start 154.8 121.77863) (end 160.05613 116.5225) (width 0.2) (layer "F.Cu") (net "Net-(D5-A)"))
 (segment (start 176.07722 103.91) (end 179.54625 100.44097) (width 0.2) (layer "B.Cu") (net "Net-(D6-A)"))
 (segment (start 173.7 103.91) (end 176.07722 103.91) (width 0.2) (layer "B.Cu") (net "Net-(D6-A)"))
 (segment (start 179.54625 100.44097) (end 179.54625 97.4725) (width 0.2) (layer "B.Cu") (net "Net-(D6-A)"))
 (segment (start 173.8 121.51) (end 178.7875 116.5225) (width 0.2) (layer "B.Cu") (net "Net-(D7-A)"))
 (segment (start 178.7875 116.5225) (end 179.54625 116.5225) (width 0.2) (layer "B.Cu") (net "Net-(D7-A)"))
 (segment (start 197.71375 96.59) (end 198.59625 97.4725) (width 0.2) (layer "F.Cu") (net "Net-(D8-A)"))
 (segment (start 193 96.59) (end 197.71375 96.59) (width 0.2) (layer "F.Cu") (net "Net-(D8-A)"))
 (segment (start 193 121.71) (end 193 120.57863) (width 0.2) (layer "F.Cu") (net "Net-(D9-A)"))
 (segment (start 197.05613 116.5225) (end 198.59625 116.5225) (width 0.2) (layer "F.Cu") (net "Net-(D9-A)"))
 (segment (start 193 120.57863) (end 197.05613 116.5225) (width 0.2) (layer "F.Cu") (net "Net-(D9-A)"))
 (segment (start 157.98 59.7) (end 166.84625 68.56625) (width 0.2) (layer "F.Cu") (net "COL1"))
 (segment (start 166.84625 68.56625) (end 166.84625 75.8825) (width 0.2) (layer "F.Cu") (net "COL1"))
 (segment (start 185.89625 75.8825) (end 204.94625 75.8825) (width 0.2) (layer "B.Cu") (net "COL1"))
 (segment (start 166.84625 75.8825) (end 185.89625 75.8825) (width 0.2) (layer "B.Cu") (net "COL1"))
 (segment (start 166.84625 94.9325) (end 204.94625 94.9325) (width 0.2) (layer "F.Cu") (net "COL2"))
 (segment (start 161.95525 66.21525) (end 161.95525 90.0415) (width 0.2) (layer "F.Cu") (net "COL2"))
 (segment (start 161.95525 90.0415) (end 166.84625 94.9325) (width 0.2) (layer "F.Cu") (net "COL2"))
 (segment (start 157.98 62.24) (end 161.95525 66.21525) (width 0.2) (layer "F.Cu") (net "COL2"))
 (segment (start 157.98 64.78) (end 159.043 65.843) (width 0.2) (layer "F.Cu") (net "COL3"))
 (segment (start 187.10475 115.191) (end 185.89625 113.9825) (width 0.2) (layer "F.Cu") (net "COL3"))
 (segment (start 204.94625 113.9825) (end 194.99366 113.9825) (width 0.2) (layer "F.Cu") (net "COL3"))
 (segment (start 158.02525 105.1615) (end 166.84625 113.9825) (width 0.2) (layer "F.Cu") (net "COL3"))
 (segment (start 194.99366 113.9825) (end 193.78516 115.191) (width 0.2) (layer "F.Cu") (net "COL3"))
 (segment (start 193.78516 115.191) (end 187.10475 115.191) (width 0.2) (layer "F.Cu") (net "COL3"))
 (segment (start 184.809 114.991) (end 167.85475 114.991) (width 0.2) (layer "F.Cu") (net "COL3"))
 (segment (start 159.043 79.44728) (end 158.02525 80.46503) (width 0.2) (layer "F.Cu") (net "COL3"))
 (segment (start 185.89625 113.9825) (end 185.8175 113.9825) (width 0.2) (layer "F.Cu") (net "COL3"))
 (segment (start 167.85475 114.991) (end 166.84625 113.9825) (width 0.2) (layer "F.Cu") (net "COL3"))
 (segment (start 185.8175 113.9825) (end 184.809 114.991) (width 0.2) (layer "F.Cu") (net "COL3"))
 (segment (start 159.043 65.843) (end 159.043 79.44728) (width 0.2) (layer "F.Cu") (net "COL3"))
 (segment (start 158.02525 80.46503) (end 158.02525 105.1615) (width 0.2) (layer "F.Cu") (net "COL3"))
 (segment (start 187.692455 56.097) (end 190.928994 59.333539) (width 0.2) (layer "B.Cu") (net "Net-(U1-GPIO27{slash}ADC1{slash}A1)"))
 (segment (start 159.457 56.097) (end 187.692455 56.097) (width 0.2) (layer "B.Cu") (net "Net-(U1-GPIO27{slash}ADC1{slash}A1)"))
 (segment (start 157.98 54.62) (end 159.457 56.097) (width 0.2) (layer "B.Cu") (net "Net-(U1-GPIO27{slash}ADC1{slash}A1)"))
 (segment (start 185.296455 48.701) (end 162.099 48.701) (width 0.2) (layer "F.Cu") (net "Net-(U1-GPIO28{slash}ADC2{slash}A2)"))
 (segment (start 162.099 48.701) (end 159.7 51.1) (width 0.2) (layer "F.Cu") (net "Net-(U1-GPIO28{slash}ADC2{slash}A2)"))
 (segment (start 159.7 55.44) (end 157.98 57.16) (width 0.2) (layer "F.Cu") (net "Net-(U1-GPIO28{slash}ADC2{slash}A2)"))
 (segment (start 190.928994 54.333539) (end 185.296455 48.701) (width 0.2) (layer "F.Cu") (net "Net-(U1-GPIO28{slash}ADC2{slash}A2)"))
 (segment (start 159.7 51.1) (end 159.7 55.44) (width 0.2) (layer "F.Cu") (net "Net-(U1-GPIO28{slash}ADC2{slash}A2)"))
 (segment (start 207.5 48.3) (end 161.76 48.3) (width 0.2) (layer "F.Cu") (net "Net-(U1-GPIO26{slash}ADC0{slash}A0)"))
 (segment (start 207.466461 59.333539) (end 207.9 58.9) (width 0.2) (layer "F.Cu") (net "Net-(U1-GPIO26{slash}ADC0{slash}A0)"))
 (segment (start 207.9 48.7) (end 207.5 48.3) (width 0.2) (layer "F.Cu") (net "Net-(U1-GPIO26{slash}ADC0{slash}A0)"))
 (segment (start 207.9 58.9) (end 207.9 48.7) (width 0.2) (layer "F.Cu") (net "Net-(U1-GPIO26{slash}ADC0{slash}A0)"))
 (segment (start 161.76 48.3) (end 157.98 52.08) (width 0.2) (layer "F.Cu") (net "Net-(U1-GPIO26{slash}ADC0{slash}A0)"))
 (segment (start 205.428994 59.333539) (end 207.466461 59.333539) (width 0.2) (layer "F.Cu") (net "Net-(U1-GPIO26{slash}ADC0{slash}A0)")))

